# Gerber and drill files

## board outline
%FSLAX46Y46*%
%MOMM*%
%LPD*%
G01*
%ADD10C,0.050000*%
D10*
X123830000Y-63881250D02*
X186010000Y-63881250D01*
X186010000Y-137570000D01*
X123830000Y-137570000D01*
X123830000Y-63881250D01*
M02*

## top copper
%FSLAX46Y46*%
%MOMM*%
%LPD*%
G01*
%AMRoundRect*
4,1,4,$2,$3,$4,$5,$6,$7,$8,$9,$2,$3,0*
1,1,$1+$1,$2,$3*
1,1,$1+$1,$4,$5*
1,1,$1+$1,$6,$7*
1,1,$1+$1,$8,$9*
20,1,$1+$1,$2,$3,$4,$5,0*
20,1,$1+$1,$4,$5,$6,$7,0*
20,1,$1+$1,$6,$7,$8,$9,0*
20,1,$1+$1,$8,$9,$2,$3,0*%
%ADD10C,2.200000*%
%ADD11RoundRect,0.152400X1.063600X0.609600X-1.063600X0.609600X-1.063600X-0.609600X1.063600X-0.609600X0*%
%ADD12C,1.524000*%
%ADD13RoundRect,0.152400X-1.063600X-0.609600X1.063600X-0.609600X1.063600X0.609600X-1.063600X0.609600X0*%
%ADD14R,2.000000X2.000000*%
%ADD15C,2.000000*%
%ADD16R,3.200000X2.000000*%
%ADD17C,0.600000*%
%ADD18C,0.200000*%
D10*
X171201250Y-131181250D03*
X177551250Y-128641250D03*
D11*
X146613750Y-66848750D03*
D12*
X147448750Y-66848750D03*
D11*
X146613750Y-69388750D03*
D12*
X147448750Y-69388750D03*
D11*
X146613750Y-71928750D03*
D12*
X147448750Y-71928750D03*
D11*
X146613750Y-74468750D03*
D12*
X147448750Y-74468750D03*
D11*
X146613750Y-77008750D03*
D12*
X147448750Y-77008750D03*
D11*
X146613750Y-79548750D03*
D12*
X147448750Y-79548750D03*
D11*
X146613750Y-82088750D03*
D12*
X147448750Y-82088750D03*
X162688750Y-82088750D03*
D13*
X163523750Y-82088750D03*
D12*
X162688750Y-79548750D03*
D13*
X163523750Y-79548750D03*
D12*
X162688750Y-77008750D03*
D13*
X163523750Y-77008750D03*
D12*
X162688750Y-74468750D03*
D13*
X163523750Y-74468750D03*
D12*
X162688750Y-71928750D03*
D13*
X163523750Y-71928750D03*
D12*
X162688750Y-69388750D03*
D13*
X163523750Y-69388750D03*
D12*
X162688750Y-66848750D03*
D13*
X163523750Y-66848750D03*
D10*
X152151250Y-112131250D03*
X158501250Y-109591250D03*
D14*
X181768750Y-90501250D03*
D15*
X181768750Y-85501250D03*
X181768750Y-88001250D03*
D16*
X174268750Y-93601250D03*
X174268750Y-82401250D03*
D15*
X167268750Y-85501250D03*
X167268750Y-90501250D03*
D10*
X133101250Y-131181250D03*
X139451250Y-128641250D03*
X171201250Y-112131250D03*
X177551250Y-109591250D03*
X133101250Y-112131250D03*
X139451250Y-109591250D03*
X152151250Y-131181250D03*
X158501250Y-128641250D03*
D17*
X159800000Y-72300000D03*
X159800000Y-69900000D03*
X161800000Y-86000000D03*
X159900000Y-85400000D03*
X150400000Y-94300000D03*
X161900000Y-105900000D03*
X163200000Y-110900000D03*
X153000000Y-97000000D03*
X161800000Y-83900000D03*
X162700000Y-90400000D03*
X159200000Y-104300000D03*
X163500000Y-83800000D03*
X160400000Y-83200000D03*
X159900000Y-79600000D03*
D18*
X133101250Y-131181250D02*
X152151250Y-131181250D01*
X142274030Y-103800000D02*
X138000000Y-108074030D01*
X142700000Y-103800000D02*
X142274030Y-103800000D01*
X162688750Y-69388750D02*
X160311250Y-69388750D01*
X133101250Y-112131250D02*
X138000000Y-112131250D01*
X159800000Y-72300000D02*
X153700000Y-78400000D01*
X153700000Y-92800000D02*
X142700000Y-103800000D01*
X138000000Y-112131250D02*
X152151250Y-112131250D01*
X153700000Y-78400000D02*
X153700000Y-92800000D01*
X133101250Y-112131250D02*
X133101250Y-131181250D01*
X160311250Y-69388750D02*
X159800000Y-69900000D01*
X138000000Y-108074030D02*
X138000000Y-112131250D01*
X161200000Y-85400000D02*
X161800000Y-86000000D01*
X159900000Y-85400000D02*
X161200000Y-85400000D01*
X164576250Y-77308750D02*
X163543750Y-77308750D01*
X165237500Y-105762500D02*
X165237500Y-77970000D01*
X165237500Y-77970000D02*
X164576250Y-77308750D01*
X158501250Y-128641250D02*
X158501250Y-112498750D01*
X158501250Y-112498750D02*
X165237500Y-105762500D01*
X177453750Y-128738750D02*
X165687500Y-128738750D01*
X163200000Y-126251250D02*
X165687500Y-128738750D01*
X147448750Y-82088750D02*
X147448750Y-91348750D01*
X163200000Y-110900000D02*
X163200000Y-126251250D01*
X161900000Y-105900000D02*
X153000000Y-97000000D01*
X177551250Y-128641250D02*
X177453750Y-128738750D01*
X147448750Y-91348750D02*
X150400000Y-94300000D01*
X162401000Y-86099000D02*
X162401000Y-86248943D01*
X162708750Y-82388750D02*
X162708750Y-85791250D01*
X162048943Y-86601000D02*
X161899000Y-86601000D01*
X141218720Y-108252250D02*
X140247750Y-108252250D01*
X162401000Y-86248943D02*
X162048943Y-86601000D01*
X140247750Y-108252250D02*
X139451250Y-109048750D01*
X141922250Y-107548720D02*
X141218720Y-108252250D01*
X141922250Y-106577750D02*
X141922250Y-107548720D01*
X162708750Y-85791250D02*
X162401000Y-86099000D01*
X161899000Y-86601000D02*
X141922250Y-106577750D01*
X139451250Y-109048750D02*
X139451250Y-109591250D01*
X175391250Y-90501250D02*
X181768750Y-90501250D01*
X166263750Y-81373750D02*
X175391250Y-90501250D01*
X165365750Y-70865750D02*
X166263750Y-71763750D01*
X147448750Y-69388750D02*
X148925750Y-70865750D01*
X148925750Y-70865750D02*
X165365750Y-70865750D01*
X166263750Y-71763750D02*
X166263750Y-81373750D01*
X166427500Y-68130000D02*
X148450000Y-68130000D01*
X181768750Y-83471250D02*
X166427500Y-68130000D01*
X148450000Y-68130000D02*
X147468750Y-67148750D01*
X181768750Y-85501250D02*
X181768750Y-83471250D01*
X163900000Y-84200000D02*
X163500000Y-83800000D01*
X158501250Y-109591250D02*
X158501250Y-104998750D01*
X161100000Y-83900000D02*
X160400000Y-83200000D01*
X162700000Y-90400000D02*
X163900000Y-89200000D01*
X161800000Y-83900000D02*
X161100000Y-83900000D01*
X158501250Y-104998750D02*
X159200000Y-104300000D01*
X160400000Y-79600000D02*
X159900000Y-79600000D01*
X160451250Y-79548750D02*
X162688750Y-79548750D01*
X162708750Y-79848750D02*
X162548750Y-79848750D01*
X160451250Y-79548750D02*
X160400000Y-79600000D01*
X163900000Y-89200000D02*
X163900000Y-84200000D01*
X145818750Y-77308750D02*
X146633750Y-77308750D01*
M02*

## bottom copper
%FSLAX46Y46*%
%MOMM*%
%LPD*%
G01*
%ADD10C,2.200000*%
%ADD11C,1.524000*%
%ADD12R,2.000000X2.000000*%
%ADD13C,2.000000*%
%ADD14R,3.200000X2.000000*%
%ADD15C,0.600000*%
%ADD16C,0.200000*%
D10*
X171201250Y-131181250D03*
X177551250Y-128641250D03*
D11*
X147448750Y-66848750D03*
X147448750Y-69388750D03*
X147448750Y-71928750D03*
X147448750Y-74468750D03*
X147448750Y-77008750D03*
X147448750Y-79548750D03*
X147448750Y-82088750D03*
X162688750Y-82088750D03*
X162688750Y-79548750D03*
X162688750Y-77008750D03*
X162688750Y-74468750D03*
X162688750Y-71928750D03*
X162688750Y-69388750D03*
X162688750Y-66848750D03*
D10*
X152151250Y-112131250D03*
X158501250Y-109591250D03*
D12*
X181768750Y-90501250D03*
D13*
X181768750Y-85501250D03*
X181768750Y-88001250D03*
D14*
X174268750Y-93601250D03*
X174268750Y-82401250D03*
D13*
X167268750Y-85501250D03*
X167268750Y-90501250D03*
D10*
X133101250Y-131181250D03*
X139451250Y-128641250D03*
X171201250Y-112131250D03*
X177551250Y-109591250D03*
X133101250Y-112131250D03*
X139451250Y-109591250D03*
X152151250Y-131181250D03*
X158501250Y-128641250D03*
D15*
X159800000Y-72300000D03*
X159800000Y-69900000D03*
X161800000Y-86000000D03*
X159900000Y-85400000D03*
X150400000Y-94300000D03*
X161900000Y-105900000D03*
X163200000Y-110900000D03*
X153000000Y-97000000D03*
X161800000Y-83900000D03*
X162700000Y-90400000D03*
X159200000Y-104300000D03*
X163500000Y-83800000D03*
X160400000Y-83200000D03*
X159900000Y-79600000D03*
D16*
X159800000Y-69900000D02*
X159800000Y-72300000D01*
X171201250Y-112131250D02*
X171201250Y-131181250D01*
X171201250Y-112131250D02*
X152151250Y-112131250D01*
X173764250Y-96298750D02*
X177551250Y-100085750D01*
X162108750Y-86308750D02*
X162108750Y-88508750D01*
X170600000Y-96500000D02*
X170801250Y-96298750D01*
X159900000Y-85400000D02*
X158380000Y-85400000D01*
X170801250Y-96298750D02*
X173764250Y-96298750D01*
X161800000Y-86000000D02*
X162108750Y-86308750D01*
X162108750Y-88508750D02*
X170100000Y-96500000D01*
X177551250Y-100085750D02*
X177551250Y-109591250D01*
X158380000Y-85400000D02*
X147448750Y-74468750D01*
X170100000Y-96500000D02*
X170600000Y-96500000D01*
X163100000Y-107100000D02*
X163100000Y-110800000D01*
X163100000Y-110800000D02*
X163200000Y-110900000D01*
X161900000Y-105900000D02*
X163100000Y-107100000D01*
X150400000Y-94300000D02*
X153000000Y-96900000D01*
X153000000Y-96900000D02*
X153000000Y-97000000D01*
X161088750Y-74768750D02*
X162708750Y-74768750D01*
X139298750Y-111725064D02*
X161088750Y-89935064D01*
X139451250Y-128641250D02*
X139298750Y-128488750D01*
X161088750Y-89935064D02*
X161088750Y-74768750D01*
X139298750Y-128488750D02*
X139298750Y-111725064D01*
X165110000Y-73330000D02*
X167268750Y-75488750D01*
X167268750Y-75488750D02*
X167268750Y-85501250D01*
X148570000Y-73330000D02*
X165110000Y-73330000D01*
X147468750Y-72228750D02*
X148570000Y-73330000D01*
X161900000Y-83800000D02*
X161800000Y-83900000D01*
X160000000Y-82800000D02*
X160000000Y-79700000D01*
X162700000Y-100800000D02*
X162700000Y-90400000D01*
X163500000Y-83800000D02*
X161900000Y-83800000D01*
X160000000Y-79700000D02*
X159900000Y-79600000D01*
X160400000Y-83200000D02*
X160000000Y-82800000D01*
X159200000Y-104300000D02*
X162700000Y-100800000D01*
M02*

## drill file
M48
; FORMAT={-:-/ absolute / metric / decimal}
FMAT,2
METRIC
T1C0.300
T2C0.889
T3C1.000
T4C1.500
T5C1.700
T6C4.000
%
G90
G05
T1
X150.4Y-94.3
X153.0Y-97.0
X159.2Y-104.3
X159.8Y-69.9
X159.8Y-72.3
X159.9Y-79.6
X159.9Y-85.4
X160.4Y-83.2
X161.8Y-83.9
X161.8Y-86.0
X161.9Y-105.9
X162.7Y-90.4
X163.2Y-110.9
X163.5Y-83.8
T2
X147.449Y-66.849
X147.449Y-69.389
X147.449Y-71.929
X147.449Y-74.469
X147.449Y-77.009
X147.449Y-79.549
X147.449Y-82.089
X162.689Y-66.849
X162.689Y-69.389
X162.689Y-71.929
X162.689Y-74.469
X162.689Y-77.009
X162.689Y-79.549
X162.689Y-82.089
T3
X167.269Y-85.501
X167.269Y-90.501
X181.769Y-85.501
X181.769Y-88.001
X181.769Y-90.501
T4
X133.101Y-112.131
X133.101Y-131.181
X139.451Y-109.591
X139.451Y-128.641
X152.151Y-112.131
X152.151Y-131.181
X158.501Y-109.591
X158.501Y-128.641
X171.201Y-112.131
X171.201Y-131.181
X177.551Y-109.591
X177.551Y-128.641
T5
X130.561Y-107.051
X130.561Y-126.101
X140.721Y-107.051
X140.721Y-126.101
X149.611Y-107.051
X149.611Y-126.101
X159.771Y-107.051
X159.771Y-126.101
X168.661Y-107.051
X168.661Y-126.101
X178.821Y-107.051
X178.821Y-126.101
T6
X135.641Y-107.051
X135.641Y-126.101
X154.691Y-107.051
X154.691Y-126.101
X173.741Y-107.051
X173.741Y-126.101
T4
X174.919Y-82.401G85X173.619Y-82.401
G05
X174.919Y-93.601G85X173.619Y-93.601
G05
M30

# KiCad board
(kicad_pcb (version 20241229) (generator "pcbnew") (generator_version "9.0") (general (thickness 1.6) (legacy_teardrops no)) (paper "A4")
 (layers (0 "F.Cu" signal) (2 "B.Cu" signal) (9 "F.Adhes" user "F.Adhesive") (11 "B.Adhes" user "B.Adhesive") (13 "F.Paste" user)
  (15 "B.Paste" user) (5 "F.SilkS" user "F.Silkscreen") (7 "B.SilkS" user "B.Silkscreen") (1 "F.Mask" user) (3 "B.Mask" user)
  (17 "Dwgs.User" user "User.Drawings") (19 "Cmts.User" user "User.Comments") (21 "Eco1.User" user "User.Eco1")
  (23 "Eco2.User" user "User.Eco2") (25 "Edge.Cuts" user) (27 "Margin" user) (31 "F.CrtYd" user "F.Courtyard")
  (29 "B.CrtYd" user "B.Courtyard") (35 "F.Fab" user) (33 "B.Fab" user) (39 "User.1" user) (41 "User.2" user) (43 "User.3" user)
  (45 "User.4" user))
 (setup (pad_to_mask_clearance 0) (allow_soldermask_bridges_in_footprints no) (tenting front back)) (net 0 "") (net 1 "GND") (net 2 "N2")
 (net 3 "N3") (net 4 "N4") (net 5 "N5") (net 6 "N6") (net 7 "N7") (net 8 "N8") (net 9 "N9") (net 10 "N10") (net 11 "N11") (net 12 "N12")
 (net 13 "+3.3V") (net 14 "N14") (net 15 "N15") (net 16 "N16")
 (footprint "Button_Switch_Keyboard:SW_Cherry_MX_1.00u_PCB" (layer "F.Cu") (at 171.20125 131.18125 180)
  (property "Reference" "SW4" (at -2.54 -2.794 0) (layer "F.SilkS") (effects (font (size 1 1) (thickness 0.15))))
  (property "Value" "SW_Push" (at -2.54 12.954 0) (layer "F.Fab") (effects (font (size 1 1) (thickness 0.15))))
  (pad "" np_thru_hole circle (at -7.62 5.08 180) (size 1.7 1.7) (drill 1.7) (layers "*.Cu" "*.Mask"))
  (pad "" np_thru_hole circle (at -2.54 5.08 180) (size 4 4) (drill 4) (layers "*.Cu" "*.Mask"))
  (pad "" np_thru_hole circle (at 2.54 5.08 180) (size 1.7 1.7) (drill 1.7) (layers "*.Cu" "*.Mask"))
  (pad "1" thru_hole circle (at 0 0 180) (size 2.2 2.2) (drill 1.5) (layers "*.Cu" "*.Mask") (remove_unused_layers no) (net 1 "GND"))
  (pad "2" thru_hole circle (at -6.35 2.54 180) (size 2.2 2.2) (drill 1.5) (layers "*.Cu" "*.Mask") (remove_unused_layers no) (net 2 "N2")))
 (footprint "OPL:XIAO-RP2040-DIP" (layer "F.Cu") (at 155.06875 74.46875)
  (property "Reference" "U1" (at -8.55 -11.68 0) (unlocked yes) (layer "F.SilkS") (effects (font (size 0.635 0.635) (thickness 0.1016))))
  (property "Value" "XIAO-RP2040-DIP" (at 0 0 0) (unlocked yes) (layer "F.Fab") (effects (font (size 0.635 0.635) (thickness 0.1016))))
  (pad "1" smd roundrect (at -8.455 -7.62 180) (size 2.432 1.524) (layers "F.Cu" "F.Mask") (roundrect_rratio 0.1) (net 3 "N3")
   (thermal_bridge_angle 45))
  (pad "1" thru_hole circle (at -7.62 -7.62 180) (size 1.524 1.524) (drill 0.889) (layers "*.Cu" "*.Mask") (remove_unused_layers no)
   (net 3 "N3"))
  (pad "2" smd roundrect (at -8.455 -5.08 180) (size 2.432 1.524) (layers "F.Cu" "F.Mask") (roundrect_rratio 0.1) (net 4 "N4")
   (thermal_bridge_angle 45))
  (pad "2" thru_hole circle (at -7.62 -5.08 180) (size 1.524 1.524) (drill 0.889) (layers "*.Cu" "*.Mask") (remove_unused_layers no)
   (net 4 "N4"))
  (pad "3" smd roundrect (at -8.455 -2.54 180) (size 2.432 1.524) (layers "F.Cu" "F.Mask") (roundrect_rratio 0.1) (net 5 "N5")
   (thermal_bridge_angle 45))
  (pad "3" thru_hole circle (at -7.62 -2.54 180) (size 1.524 1.524) (drill 0.889) (layers "*.Cu" "*.Mask") (remove_unused_layers no)
   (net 5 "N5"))
  (pad "4" smd roundrect (at -8.455 0 180) (size 2.432 1.524) (layers "F.Cu" "F.Mask") (roundrect_rratio 0.1) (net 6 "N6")
   (thermal_bridge_angle 45))
  (pad "4" thru_hole circle (at -7.62 0 180) (size 1.524 1.524) (drill 0.889) (layers "*.Cu" "*.Mask") (remove_unused_layers no)
   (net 6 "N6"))
  (pad "5" smd roundrect (at -8.455 2.54 180) (size 2.432 1.524) (layers "F.Cu" "F.Mask") (roundrect_rratio 0.1) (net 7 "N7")
   (thermal_bridge_angle 45))
  (pad "5" thru_hole circle (at -7.62 2.54 180) (size 1.524 1.524) (drill 0.889) (layers "*.Cu" "*.Mask") (remove_unused_layers no)
   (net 7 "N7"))
  (pad "6" smd roundrect (at -8.455 5.08 180) (size 2.432 1.524) (layers "F.Cu" "F.Mask") (roundrect_rratio 0.1) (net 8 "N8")
   (thermal_bridge_angle 45))
  (pad "6" thru_hole circle (at -7.62 5.08 180) (size 1.524 1.524) (drill 0.889) (layers "*.Cu" "*.Mask") (remove_unused_layers no)
   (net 8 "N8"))
  (pad "7" smd roundrect (at -8.455 7.62 180) (size 2.432 1.524) (layers "F.Cu" "F.Mask") (roundrect_rratio 0.1) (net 2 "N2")
   (thermal_bridge_angle 45))
  (pad "7" thru_hole circle (at -7.62 7.62 180) (size 1.524 1.524) (drill 0.889) (layers "*.Cu" "*.Mask") (remove_unused_layers no)
   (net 2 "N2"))
  (pad "8" thru_hole circle (at 7.62 7.62) (size 1.524 1.524) (drill 0.889) (layers "*.Cu" "*.Mask") (remove_unused_layers no) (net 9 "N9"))
  (pad "8" smd roundrect (at 8.455 7.62) (size 2.432 1.524) (layers "F.Cu" "F.Mask") (roundrect_rratio 0.1) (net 9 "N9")
   (thermal_bridge_angle 45))
  (pad "9" thru_hole circle (at 7.62 5.08) (size 1.524 1.524) (drill 0.889) (layers "*.Cu" "*.Mask") (remove_unused_layers no)
   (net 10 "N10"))
  (pad "9" smd roundrect (at 8.455 5.08) (size 2.432 1.524) (layers "F.Cu" "F.Mask") (roundrect_rratio 0.1) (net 10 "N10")
   (thermal_bridge_angle 45))
  (pad "10" thru_hole circle (at 7.62 2.54) (size 1.524 1.524) (drill 0.889) (layers "*.Cu" "*.Mask") (remove_unused_layers no)
   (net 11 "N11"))
  (pad "10" smd roundrect (at 8.455 2.54) (size 2.432 1.524) (layers "F.Cu" "F.Mask") (roundrect_rratio 0.1) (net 11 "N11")
   (thermal_bridge_angle 45))
  (pad "11" thru_hole circle (at 7.62 0) (size 1.524 1.524) (drill 0.889) (layers "*.Cu" "*.Mask") (remove_unused_layers no) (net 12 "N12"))
  (pad "11" smd roundrect (at 8.455 0) (size 2.432 1.524) (layers "F.Cu" "F.Mask") (roundrect_rratio 0.1) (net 12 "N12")
   (thermal_bridge_angle 45))
  (pad "12" thru_hole circle (at 7.62 -2.54) (size 1.524 1.524) (drill 0.889) (layers "*.Cu" "*.Mask") (remove_unused_layers no)
   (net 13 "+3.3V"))
  (pad "12" smd roundrect (at 8.455 -2.54) (size 2.432 1.524) (layers "F.Cu" "F.Mask") (roundrect_rratio 0.1) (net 13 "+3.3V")
   (thermal_bridge_angle 45))
  (pad "13" thru_hole circle (at 7.62 -5.08) (size 1.524 1.524) (drill 0.889) (layers "*.Cu" "*.Mask") (remove_unused_layers no)
   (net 1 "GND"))
  (pad "13" smd roundrect (at 8.455 -5.08) (size 2.432 1.524) (layers "F.Cu" "F.Mask") (roundrect_rratio 0.1) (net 1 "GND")
   (thermal_bridge_angle 45))
  (pad "14" thru_hole circle (at 7.62 -7.62) (size 1.524 1.524) (drill 0.889) (layers "*.Cu" "*.Mask") (remove_unused_layers no)
   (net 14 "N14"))
  (pad "14" smd roundrect (at 8.455 -7.62) (size 2.432 1.524) (layers "F.Cu" "F.Mask") (roundrect_rratio 0.1) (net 14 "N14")
   (thermal_bridge_angle 45)))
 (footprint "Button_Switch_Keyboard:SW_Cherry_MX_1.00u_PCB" (layer "F.Cu") (at 152.15125 112.13125 180)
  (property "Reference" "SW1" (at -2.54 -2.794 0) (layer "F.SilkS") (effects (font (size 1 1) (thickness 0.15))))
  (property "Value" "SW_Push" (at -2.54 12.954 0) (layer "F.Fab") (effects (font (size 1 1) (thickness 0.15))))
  (pad "" np_thru_hole circle (at -7.62 5.08 180) (size 1.7 1.7) (drill 1.7) (layers "*.Cu" "*.Mask"))
  (pad "" np_thru_hole circle (at -2.54 5.08 180) (size 4 4) (drill 4) (layers "*.Cu" "*.Mask"))
  (pad "" np_thru_hole circle (at 2.54 5.08 180) (size 1.7 1.7) (drill 1.7) (layers "*.Cu" "*.Mask"))
  (pad "1" thru_hole circle (at 0 0 180) (size 2.2 2.2) (drill 1.5) (layers "*.Cu" "*.Mask") (remove_unused_layers no) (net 1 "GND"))
  (pad "2" thru_hole circle (at -6.35 2.54 180) (size 2.2 2.2) (drill 1.5) (layers "*.Cu" "*.Mask") (remove_unused_layers no) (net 10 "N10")))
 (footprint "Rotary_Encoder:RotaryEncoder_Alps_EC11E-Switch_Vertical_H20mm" (layer "F.Cu") (at 181.76875 90.50125 180)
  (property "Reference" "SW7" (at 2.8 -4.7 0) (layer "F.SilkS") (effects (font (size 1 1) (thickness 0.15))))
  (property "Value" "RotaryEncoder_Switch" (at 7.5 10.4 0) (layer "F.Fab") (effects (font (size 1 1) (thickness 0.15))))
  (pad "A" thru_hole rect (at 0 0 180) (size 2 2) (drill 1) (layers "*.Cu" "*.Mask") (remove_unused_layers no) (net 4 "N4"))
  (pad "B" thru_hole circle (at 0 5 180) (size 2 2) (drill 1) (layers "*.Cu" "*.Mask") (remove_unused_layers no) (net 3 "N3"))
  (pad "C" thru_hole circle (at 0 2.5 180) (size 2 2) (drill 1) (layers "*.Cu" "*.Mask") (remove_unused_layers no) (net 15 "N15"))
  (pad "MP" thru_hole rect (at 7.5 -3.1 180) (size 3.2 2) (drill oval 2.8 1.5) (layers "*.Cu" "*.Mask") (remove_unused_layers no))
  (pad "MP" thru_hole rect (at 7.5 8.1 180) (size 3.2 2) (drill oval 2.8 1.5) (layers "*.Cu" "*.Mask") (remove_unused_layers no))
  (pad "S1" thru_hole circle (at 14.5 5 180) (size 2 2) (drill 1) (layers "*.Cu" "*.Mask") (remove_unused_layers no) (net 5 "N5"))
  (pad "S2" thru_hole circle (at 14.5 0 180) (size 2 2) (drill 1) (layers "*.Cu" "*.Mask") (remove_unused_layers no) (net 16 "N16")))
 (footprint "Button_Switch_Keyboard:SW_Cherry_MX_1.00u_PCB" (layer "F.Cu") (at 133.10125 131.18125 180)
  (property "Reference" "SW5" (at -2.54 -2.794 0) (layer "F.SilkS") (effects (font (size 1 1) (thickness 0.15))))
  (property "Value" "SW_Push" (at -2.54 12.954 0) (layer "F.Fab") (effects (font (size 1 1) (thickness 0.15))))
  (pad "" np_thru_hole circle (at -7.62 5.08 180) (size 1.7 1.7) (drill 1.7) (layers "*.Cu" "*.Mask"))
  (pad "" np_thru_hole circle (at -2.54 5.08 180) (size 4 4) (drill 4) (layers "*.Cu" "*.Mask"))
  (pad "" np_thru_hole circle (at 2.54 5.08 180) (size 1.7 1.7) (drill 1.7) (layers "*.Cu" "*.Mask"))
  (pad "1" thru_hole circle (at 0 0 180) (size 2.2 2.2) (drill 1.5) (layers "*.Cu" "*.Mask") (remove_unused_layers no) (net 1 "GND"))
  (pad "2" thru_hole circle (at -6.35 2.54 180) (size 2.2 2.2) (drill 1.5) (layers "*.Cu" "*.Mask") (remove_unused_layers no) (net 12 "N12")))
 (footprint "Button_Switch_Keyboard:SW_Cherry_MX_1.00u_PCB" (layer "F.Cu") (at 171.20125 112.13125 180)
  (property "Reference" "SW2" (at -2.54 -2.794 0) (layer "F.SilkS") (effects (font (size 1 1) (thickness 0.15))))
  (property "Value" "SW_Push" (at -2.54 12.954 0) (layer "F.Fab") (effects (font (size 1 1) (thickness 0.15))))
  (pad "" np_thru_hole circle (at -7.62 5.08 180) (size 1.7 1.7) (drill 1.7) (layers "*.Cu" "*.Mask"))
  (pad "" np_thru_hole circle (at -2.54 5.08 180) (size 4 4) (drill 4) (layers "*.Cu" "*.Mask"))
  (pad "" np_thru_hole circle (at 2.54 5.08 180) (size 1.7 1.7) (drill 1.7) (layers "*.Cu" "*.Mask"))
  (pad "1" thru_hole circle (at 0 0 180) (size 2.2 2.2) (drill 1.5) (layers "*.Cu" "*.Mask") (remove_unused_layers no) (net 1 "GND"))
  (pad "2" thru_hole circle (at -6.35 2.54 180) (size 2.2 2.2) (drill 1.5) (layers "*.Cu" "*.Mask") (remove_unused_layers no) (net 6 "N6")))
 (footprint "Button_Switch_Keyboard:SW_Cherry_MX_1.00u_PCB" (layer "F.Cu") (at 133.10125 112.13125 180)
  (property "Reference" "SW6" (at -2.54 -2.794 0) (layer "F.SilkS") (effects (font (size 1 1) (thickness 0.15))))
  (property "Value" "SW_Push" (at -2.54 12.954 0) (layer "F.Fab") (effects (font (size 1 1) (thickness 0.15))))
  (pad "" np_thru_hole circle (at -7.62 5.08 180) (size 1.7 1.7) (drill 1.7) (layers "*.Cu" "*.Mask"))
  (pad "" np_thru_hole circle (at -2.54 5.08 180) (size 4 4) (drill 4) (layers "*.Cu" "*.Mask"))
  (pad "" np_thru_hole circle (at 2.54 5.08 180) (size 1.7 1.7) (drill 1.7) (layers "*.Cu" "*.Mask"))
  (pad "1" thru_hole circle (at 0 0 180) (size 2.2 2.2) (drill 1.5) (layers "*.Cu" "*.Mask") (remove_unused_layers no) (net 1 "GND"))
  (pad "2" thru_hole circle (at -6.35 2.54 180) (size 2.2 2.2) (drill 1.5) (layers "*.Cu" "*.Mask") (remove_unused_layers no) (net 9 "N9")))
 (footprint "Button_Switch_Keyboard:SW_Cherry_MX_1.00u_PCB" (layer "F.Cu") (at 152.15125 131.18125 180)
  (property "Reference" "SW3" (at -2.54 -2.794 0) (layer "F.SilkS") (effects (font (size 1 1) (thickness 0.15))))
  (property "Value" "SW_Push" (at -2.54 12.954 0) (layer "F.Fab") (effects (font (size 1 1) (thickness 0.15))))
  (pad "" np_thru_hole circle (at -7.62 5.08 180) (size 1.7 1.7) (drill 1.7) (layers "*.Cu" "*.Mask"))
  (pad "" np_thru_hole circle (at -2.54 5.08 180) (size 4 4) (drill 4) (layers "*.Cu" "*.Mask"))
  (pad "" np_thru_hole circle (at 2.54 5.08 180) (size 1.7 1.7) (drill 1.7) (layers "*.Cu" "*.Mask"))
  (pad "1" thru_hole circle (at 0 0 180) (size 2.2 2.2) (drill 1.5) (layers "*.Cu" "*.Mask") (remove_unused_layers no) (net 1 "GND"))
  (pad "2" thru_hole circle (at -6.35 2.54 180) (size 2.2 2.2) (drill 1.5) (layers "*.Cu" "*.Mask") (remove_unused_layers no) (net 11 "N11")))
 (gr_rect (start 123.83 63.88125) (end 186.01 137.57) (stroke (width 0.05) (type default)) (fill no) (layer "Edge.Cuts"))
 (segment (start 133.10125 131.18125) (end 152.15125 131.18125) (width 0.2) (layer "F.Cu") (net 1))
 (segment (start 142.27403 103.8) (end 138 108.07403) (width 0.2) (layer "F.Cu") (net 1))
 (segment (start 142.7 103.8) (end 142.27403 103.8) (width 0.2) (layer "F.Cu") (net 1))
 (segment (start 162.68875 69.38875) (end 160.31125 69.38875) (width 0.2) (layer "F.Cu") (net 1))
 (segment (start 133.10125 112.13125) (end 138 112.13125) (width 0.2) (layer "F.Cu") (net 1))
 (segment (start 159.8 72.3) (end 153.7 78.4) (width 0.2) (layer "F.Cu") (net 1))
 (segment (start 153.7 92.8) (end 142.7 103.8) (width 0.2) (layer "F.Cu") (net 1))
 (segment (start 138 112.13125) (end 152.15125 112.13125) (width 0.2) (layer "F.Cu") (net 1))
 (segment (start 153.7 78.4) (end 153.7 92.8) (width 0.2) (layer "F.Cu") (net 1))
 (segment (start 133.10125 112.13125) (end 133.10125 131.18125) (width 0.2) (layer "F.Cu") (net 1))
 (segment (start 160.31125 69.38875) (end 159.8 69.9) (width 0.2) (layer "F.Cu") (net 1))
 (segment (start 138 108.07403) (end 138 112.13125) (width 0.2) (layer "F.Cu") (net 1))
 (via (at 159.8 72.3) (size 0.6) (drill 0.3) (layers "F.Cu" "B.Cu") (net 1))
 (via (at 159.8 69.9) (size 0.6) (drill 0.3) (layers "F.Cu" "B.Cu") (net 1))
 (segment (start 159.8 69.9) (end 159.8 72.3) (width 0.2) (layer "B.Cu") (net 1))
 (segment (start 171.20125 112.13125) (end 171.20125 131.18125) (width 0.2) (layer "B.Cu") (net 1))
 (segment (start 171.20125 112.13125) (end 152.15125 112.13125) (width 0.2) (layer "B.Cu") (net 1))
 (segment (start 161.2 85.4) (end 161.8 86) (width 0.2) (layer "F.Cu") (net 6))
 (segment (start 159.9 85.4) (end 161.2 85.4) (width 0.2) (layer "F.Cu") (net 6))
 (via (at 161.8 86) (size 0.6) (drill 0.3) (layers "F.Cu" "B.Cu") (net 6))
 (via (at 159.9 85.4) (size 0.6) (drill 0.3) (layers "F.Cu" "B.Cu") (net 6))
 (segment (start 173.76425 96.29875) (end 177.55125 100.08575) (width 0.2) (layer "B.Cu") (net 6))
 (segment (start 162.10875 86.30875) (end 162.10875 88.50875) (width 0.2) (layer "B.Cu") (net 6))
 (segment (start 170.6 96.5) (end 170.80125 96.29875) (width 0.2) (layer "B.Cu") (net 6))
 (segment (start 159.9 85.4) (end 158.38 85.4) (width 0.2) (layer "B.Cu") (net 6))
 (segment (start 170.80125 96.29875) (end 173.76425 96.29875) (width 0.2) (layer "B.Cu") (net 6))
 (segment (start 161.8 86) (end 162.10875 86.30875) (width 0.2) (layer "B.Cu") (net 6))
 (segment (start 162.10875 88.50875) (end 170.1 96.5) (width 0.2) (layer "B.Cu") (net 6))
 (segment (start 177.55125 100.08575) (end 177.55125 109.59125) (width 0.2) (layer "B.Cu") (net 6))
 (segment (start 158.38 85.4) (end 147.44875 74.46875) (width 0.2) (layer "B.Cu") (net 6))
 (segment (start 170.1 96.5) (end 170.6 96.5) (width 0.2) (layer "B.Cu") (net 6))
 (segment (start 164.57625 77.30875) (end 163.54375 77.30875) (width 0.2) (layer "F.Cu") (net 11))
 (segment (start 165.2375 105.7625) (end 165.2375 77.97) (width 0.2) (layer "F.Cu") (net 11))
 (segment (start 165.2375 77.97) (end 164.57625 77.30875) (width 0.2) (layer "F.Cu") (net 11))
 (segment (start 158.50125 128.64125) (end 158.50125 112.49875) (width 0.2) (layer "F.Cu") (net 11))
 (segment (start 158.50125 112.49875) (end 165.2375 105.7625) (width 0.2) (layer "F.Cu") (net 11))
 (segment (start 177.45375 128.73875) (end 165.6875 128.73875) (width 0.2) (layer "F.Cu") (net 2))
 (segment (start 163.2 126.25125) (end 165.6875 128.73875) (width 0.2) (layer "F.Cu") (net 2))
 (segment (start 147.44875 82.08875) (end 147.44875 91.34875) (width 0.2) (layer "F.Cu") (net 2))
 (segment (start 163.2 110.9) (end 163.2 126.25125) (width 0.2) (layer "F.Cu") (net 2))
 (segment (start 161.9 105.9) (end 153 97) (width 0.2) (layer "F.Cu") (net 2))
 (segment (start 177.55125 128.64125) (end 177.45375 128.73875) (width 0.2) (layer "F.Cu") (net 2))
 (segment (start 147.44875 91.34875) (end 150.4 94.3) (width 0.2) (layer "F.Cu") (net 2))
 (via (at 150.4 94.3) (size 0.6) (drill 0.3) (layers "F.Cu" "B.Cu") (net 2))
 (via (at 161.9 105.9) (size 0.6) (drill 0.3) (layers "F.Cu" "B.Cu") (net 2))
 (via (at 163.2 110.9) (size 0.6) (drill 0.3) (layers "F.Cu" "B.Cu") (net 2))
 (via (at 153 97) (size 0.6) (drill 0.3) (layers "F.Cu" "B.Cu") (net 2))
 (segment (start 163.1 107.1) (end 163.1 110.8) (width 0.2) (layer "B.Cu") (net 2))
 (segment (start 163.1 110.8) (end 163.2 110.9) (width 0.2) (layer "B.Cu") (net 2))
 (segment (start 161.9 105.9) (end 163.1 107.1) (width 0.2) (layer "B.Cu") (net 2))
 (segment (start 150.4 94.3) (end 153 96.9) (width 0.2) (layer "B.Cu") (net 2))
 (segment (start 153 96.9) (end 153 97) (width 0.2) (layer "B.Cu") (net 2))
 (segment (start 161.08875 74.76875) (end 162.70875 74.76875) (width 0.2) (layer "B.Cu") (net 12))
 (segment (start 139.29875 111.725064) (end 161.08875 89.935064) (width 0.2) (layer "B.Cu") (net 12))
 (segment (start 139.45125 128.64125) (end 139.29875 128.48875) (width 0.2) (layer "B.Cu") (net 12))
 (segment (start 161.08875 89.935064) (end 161.08875 74.76875) (width 0.2) (layer "B.Cu") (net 12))
 (segment (start 139.29875 128.48875) (end 139.29875 111.725064) (width 0.2) (layer "B.Cu") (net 12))
 (segment (start 162.401 86.099) (end 162.401 86.248943) (width 0.2) (layer "F.Cu") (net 9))
 (segment (start 162.70875 82.38875) (end 162.70875 85.79125) (width 0.2) (layer "F.Cu") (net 9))
 (segment (start 162.048943 86.601) (end 161.899 86.601) (width 0.2) (layer "F.Cu") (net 9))
 (segment (start 141.21872 108.25225) (end 140.24775 108.25225) (width 0.2) (layer "F.Cu") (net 9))
 (segment (start 162.401 86.248943) (end 162.048943 86.601) (width 0.2) (layer "F.Cu") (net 9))
 (segment (start 140.24775 108.25225) (end 139.45125 109.04875) (width 0.2) (layer "F.Cu") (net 9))
 (segment (start 141.92225 107.54872) (end 141.21872 108.25225) (width 0.2) (layer "F.Cu") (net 9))
 (segment (start 141.92225 106.57775) (end 141.92225 107.54872) (width 0.2) (layer "F.Cu") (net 9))
 (segment (start 162.70875 85.79125) (end 162.401 86.099) (width 0.2) (layer "F.Cu") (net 9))
 (segment (start 161.899 86.601) (end 141.92225 106.57775) (width 0.2) (layer "F.Cu") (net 9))
 (segment (start 139.45125 109.04875) (end 139.45125 109.59125) (width 0.2) (layer "F.Cu") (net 9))
 (segment (start 165.11 73.33) (end 167.26875 75.48875) (width 0.2) (layer "B.Cu") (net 5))
 (segment (start 167.26875 75.48875) (end 167.26875 85.50125) (width 0.2) (layer "B.Cu") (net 5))
 (segment (start 148.57 73.33) (end 165.11 73.33) (width 0.2) (layer "B.Cu") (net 5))
 (segment (start 147.46875 72.22875) (end 148.57 73.33) (width 0.2) (layer "B.Cu") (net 5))
 (segment (start 175.39125 90.50125) (end 181.76875 90.50125) (width 0.2) (layer "F.Cu") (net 4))
 (segment (start 166.26375 81.37375) (end 175.39125 90.50125) (width 0.2) (layer "F.Cu") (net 4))
 (segment (start 165.36575 70.86575) (end 166.26375 71.76375) (width 0.2) (layer "F.Cu") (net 4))
 (segment (start 147.44875 69.38875) (end 148.92575 70.86575) (width 0.2) (layer "F.Cu") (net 4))
 (segment (start 148.92575 70.86575) (end 165.36575 70.86575) (width 0.2) (layer "F.Cu") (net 4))
 (segment (start 166.26375 71.76375) (end 166.26375 81.37375) (width 0.2) (layer "F.Cu") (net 4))
 (segment (start 166.4275 68.13) (end 148.45 68.13) (width 0.2) (layer "F.Cu") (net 3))
 (segment (start 181.76875 83.47125) (end 166.4275 68.13) (width 0.2) (layer "F.Cu") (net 3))
 (segment (start 148.45 68.13) (end 147.46875 67.14875) (width 0.2) (layer "F.Cu") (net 3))
 (segment (start 181.76875 85.50125) (end 181.76875 83.47125) (width 0.2) (layer "F.Cu") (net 3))
 (segment (start 163.9 84.2) (end 163.5 83.8) (width 0.2) (layer "F.Cu") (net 10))
 (segment (start 158.50125 109.59125) (end 158.50125 104.99875) (width 0.2) (layer "F.Cu") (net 10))
 (segment (start 161.1 83.9) (end 160.4 83.2) (width 0.2) (layer "F.Cu") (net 10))
 (segment (start 162.7 90.4) (end 163.9 89.2) (width 0.2) (layer "F.Cu") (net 10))
 (segment (start 161.8 83.9) (end 161.1 83.9) (width 0.2) (layer "F.Cu") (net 10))
 (segment (start 158.50125 104.99875) (end 159.2 104.3) (width 0.2) (layer "F.Cu") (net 10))
 (segment (start 160.4 79.6) (end 159.9 79.6) (width 0.2) (layer "F.Cu") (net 10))
 (segment (start 160.45125 79.54875) (end 162.68875 79.54875) (width 0.2) (layer "F.Cu") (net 10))
 (segment (start 162.70875 79.84875) (end 162.54875 79.84875) (width 0.2) (layer "F.Cu") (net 10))
 (segment (start 160.45125 79.54875) (end 160.4 79.6) (width 0.2) (layer "F.Cu") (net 10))
 (segment (start 163.9 89.2) (end 163.9 84.2) (width 0.2) (layer "F.Cu") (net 10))
 (via (at 161.8 83.9) (size 0.6) (drill 0.3) (layers "F.Cu" "B.Cu") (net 10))
 (via (at 162.7 90.4) (size 0.6) (drill 0.3) (layers "F.Cu" "B.Cu") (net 10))
 (via (at 159.2 104.3) (size 0.6) (drill 0.3) (layers "F.Cu" "B.Cu") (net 10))
 (via (at 163.5 83.8) (size 0.6) (drill 0.3) (layers "F.Cu" "B.Cu") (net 10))
 (via (at 160.4 83.2) (size 0.6) (drill 0.3) (layers "F.Cu" "B.Cu") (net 10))
 (via (at 159.9 79.6) (size 0.6) (drill 0.3) (layers "F.Cu" "B.Cu") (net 10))
 (segment (start 161.9 83.8) (end 161.8 83.9) (width 0.2) (layer "B.Cu") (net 10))
 (segment (start 160 82.8) (end 160 79.7) (width 0.2) (layer "B.Cu") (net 10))
 (segment (start 162.7 100.8) (end 162.7 90.4) (width 0.2) (layer "B.Cu") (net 10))
 (segment (start 163.5 83.8) (end 161.9 83.8) (width 0.2) (layer "B.Cu") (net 10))
 (segment (start 160 79.7) (end 159.9 79.6) (width 0.2) (layer "B.Cu") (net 10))
 (segment (start 160.4 83.2) (end 160 82.8) (width 0.2) (layer "B.Cu") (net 10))
 (segment (start 159.2 104.3) (end 162.7 100.8) (width 0.2) (layer "B.Cu") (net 10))
 (segment (start 145.81875 77.30875) (end 146.63375 77.30875) (width 0.2) (layer "F.Cu") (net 7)))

